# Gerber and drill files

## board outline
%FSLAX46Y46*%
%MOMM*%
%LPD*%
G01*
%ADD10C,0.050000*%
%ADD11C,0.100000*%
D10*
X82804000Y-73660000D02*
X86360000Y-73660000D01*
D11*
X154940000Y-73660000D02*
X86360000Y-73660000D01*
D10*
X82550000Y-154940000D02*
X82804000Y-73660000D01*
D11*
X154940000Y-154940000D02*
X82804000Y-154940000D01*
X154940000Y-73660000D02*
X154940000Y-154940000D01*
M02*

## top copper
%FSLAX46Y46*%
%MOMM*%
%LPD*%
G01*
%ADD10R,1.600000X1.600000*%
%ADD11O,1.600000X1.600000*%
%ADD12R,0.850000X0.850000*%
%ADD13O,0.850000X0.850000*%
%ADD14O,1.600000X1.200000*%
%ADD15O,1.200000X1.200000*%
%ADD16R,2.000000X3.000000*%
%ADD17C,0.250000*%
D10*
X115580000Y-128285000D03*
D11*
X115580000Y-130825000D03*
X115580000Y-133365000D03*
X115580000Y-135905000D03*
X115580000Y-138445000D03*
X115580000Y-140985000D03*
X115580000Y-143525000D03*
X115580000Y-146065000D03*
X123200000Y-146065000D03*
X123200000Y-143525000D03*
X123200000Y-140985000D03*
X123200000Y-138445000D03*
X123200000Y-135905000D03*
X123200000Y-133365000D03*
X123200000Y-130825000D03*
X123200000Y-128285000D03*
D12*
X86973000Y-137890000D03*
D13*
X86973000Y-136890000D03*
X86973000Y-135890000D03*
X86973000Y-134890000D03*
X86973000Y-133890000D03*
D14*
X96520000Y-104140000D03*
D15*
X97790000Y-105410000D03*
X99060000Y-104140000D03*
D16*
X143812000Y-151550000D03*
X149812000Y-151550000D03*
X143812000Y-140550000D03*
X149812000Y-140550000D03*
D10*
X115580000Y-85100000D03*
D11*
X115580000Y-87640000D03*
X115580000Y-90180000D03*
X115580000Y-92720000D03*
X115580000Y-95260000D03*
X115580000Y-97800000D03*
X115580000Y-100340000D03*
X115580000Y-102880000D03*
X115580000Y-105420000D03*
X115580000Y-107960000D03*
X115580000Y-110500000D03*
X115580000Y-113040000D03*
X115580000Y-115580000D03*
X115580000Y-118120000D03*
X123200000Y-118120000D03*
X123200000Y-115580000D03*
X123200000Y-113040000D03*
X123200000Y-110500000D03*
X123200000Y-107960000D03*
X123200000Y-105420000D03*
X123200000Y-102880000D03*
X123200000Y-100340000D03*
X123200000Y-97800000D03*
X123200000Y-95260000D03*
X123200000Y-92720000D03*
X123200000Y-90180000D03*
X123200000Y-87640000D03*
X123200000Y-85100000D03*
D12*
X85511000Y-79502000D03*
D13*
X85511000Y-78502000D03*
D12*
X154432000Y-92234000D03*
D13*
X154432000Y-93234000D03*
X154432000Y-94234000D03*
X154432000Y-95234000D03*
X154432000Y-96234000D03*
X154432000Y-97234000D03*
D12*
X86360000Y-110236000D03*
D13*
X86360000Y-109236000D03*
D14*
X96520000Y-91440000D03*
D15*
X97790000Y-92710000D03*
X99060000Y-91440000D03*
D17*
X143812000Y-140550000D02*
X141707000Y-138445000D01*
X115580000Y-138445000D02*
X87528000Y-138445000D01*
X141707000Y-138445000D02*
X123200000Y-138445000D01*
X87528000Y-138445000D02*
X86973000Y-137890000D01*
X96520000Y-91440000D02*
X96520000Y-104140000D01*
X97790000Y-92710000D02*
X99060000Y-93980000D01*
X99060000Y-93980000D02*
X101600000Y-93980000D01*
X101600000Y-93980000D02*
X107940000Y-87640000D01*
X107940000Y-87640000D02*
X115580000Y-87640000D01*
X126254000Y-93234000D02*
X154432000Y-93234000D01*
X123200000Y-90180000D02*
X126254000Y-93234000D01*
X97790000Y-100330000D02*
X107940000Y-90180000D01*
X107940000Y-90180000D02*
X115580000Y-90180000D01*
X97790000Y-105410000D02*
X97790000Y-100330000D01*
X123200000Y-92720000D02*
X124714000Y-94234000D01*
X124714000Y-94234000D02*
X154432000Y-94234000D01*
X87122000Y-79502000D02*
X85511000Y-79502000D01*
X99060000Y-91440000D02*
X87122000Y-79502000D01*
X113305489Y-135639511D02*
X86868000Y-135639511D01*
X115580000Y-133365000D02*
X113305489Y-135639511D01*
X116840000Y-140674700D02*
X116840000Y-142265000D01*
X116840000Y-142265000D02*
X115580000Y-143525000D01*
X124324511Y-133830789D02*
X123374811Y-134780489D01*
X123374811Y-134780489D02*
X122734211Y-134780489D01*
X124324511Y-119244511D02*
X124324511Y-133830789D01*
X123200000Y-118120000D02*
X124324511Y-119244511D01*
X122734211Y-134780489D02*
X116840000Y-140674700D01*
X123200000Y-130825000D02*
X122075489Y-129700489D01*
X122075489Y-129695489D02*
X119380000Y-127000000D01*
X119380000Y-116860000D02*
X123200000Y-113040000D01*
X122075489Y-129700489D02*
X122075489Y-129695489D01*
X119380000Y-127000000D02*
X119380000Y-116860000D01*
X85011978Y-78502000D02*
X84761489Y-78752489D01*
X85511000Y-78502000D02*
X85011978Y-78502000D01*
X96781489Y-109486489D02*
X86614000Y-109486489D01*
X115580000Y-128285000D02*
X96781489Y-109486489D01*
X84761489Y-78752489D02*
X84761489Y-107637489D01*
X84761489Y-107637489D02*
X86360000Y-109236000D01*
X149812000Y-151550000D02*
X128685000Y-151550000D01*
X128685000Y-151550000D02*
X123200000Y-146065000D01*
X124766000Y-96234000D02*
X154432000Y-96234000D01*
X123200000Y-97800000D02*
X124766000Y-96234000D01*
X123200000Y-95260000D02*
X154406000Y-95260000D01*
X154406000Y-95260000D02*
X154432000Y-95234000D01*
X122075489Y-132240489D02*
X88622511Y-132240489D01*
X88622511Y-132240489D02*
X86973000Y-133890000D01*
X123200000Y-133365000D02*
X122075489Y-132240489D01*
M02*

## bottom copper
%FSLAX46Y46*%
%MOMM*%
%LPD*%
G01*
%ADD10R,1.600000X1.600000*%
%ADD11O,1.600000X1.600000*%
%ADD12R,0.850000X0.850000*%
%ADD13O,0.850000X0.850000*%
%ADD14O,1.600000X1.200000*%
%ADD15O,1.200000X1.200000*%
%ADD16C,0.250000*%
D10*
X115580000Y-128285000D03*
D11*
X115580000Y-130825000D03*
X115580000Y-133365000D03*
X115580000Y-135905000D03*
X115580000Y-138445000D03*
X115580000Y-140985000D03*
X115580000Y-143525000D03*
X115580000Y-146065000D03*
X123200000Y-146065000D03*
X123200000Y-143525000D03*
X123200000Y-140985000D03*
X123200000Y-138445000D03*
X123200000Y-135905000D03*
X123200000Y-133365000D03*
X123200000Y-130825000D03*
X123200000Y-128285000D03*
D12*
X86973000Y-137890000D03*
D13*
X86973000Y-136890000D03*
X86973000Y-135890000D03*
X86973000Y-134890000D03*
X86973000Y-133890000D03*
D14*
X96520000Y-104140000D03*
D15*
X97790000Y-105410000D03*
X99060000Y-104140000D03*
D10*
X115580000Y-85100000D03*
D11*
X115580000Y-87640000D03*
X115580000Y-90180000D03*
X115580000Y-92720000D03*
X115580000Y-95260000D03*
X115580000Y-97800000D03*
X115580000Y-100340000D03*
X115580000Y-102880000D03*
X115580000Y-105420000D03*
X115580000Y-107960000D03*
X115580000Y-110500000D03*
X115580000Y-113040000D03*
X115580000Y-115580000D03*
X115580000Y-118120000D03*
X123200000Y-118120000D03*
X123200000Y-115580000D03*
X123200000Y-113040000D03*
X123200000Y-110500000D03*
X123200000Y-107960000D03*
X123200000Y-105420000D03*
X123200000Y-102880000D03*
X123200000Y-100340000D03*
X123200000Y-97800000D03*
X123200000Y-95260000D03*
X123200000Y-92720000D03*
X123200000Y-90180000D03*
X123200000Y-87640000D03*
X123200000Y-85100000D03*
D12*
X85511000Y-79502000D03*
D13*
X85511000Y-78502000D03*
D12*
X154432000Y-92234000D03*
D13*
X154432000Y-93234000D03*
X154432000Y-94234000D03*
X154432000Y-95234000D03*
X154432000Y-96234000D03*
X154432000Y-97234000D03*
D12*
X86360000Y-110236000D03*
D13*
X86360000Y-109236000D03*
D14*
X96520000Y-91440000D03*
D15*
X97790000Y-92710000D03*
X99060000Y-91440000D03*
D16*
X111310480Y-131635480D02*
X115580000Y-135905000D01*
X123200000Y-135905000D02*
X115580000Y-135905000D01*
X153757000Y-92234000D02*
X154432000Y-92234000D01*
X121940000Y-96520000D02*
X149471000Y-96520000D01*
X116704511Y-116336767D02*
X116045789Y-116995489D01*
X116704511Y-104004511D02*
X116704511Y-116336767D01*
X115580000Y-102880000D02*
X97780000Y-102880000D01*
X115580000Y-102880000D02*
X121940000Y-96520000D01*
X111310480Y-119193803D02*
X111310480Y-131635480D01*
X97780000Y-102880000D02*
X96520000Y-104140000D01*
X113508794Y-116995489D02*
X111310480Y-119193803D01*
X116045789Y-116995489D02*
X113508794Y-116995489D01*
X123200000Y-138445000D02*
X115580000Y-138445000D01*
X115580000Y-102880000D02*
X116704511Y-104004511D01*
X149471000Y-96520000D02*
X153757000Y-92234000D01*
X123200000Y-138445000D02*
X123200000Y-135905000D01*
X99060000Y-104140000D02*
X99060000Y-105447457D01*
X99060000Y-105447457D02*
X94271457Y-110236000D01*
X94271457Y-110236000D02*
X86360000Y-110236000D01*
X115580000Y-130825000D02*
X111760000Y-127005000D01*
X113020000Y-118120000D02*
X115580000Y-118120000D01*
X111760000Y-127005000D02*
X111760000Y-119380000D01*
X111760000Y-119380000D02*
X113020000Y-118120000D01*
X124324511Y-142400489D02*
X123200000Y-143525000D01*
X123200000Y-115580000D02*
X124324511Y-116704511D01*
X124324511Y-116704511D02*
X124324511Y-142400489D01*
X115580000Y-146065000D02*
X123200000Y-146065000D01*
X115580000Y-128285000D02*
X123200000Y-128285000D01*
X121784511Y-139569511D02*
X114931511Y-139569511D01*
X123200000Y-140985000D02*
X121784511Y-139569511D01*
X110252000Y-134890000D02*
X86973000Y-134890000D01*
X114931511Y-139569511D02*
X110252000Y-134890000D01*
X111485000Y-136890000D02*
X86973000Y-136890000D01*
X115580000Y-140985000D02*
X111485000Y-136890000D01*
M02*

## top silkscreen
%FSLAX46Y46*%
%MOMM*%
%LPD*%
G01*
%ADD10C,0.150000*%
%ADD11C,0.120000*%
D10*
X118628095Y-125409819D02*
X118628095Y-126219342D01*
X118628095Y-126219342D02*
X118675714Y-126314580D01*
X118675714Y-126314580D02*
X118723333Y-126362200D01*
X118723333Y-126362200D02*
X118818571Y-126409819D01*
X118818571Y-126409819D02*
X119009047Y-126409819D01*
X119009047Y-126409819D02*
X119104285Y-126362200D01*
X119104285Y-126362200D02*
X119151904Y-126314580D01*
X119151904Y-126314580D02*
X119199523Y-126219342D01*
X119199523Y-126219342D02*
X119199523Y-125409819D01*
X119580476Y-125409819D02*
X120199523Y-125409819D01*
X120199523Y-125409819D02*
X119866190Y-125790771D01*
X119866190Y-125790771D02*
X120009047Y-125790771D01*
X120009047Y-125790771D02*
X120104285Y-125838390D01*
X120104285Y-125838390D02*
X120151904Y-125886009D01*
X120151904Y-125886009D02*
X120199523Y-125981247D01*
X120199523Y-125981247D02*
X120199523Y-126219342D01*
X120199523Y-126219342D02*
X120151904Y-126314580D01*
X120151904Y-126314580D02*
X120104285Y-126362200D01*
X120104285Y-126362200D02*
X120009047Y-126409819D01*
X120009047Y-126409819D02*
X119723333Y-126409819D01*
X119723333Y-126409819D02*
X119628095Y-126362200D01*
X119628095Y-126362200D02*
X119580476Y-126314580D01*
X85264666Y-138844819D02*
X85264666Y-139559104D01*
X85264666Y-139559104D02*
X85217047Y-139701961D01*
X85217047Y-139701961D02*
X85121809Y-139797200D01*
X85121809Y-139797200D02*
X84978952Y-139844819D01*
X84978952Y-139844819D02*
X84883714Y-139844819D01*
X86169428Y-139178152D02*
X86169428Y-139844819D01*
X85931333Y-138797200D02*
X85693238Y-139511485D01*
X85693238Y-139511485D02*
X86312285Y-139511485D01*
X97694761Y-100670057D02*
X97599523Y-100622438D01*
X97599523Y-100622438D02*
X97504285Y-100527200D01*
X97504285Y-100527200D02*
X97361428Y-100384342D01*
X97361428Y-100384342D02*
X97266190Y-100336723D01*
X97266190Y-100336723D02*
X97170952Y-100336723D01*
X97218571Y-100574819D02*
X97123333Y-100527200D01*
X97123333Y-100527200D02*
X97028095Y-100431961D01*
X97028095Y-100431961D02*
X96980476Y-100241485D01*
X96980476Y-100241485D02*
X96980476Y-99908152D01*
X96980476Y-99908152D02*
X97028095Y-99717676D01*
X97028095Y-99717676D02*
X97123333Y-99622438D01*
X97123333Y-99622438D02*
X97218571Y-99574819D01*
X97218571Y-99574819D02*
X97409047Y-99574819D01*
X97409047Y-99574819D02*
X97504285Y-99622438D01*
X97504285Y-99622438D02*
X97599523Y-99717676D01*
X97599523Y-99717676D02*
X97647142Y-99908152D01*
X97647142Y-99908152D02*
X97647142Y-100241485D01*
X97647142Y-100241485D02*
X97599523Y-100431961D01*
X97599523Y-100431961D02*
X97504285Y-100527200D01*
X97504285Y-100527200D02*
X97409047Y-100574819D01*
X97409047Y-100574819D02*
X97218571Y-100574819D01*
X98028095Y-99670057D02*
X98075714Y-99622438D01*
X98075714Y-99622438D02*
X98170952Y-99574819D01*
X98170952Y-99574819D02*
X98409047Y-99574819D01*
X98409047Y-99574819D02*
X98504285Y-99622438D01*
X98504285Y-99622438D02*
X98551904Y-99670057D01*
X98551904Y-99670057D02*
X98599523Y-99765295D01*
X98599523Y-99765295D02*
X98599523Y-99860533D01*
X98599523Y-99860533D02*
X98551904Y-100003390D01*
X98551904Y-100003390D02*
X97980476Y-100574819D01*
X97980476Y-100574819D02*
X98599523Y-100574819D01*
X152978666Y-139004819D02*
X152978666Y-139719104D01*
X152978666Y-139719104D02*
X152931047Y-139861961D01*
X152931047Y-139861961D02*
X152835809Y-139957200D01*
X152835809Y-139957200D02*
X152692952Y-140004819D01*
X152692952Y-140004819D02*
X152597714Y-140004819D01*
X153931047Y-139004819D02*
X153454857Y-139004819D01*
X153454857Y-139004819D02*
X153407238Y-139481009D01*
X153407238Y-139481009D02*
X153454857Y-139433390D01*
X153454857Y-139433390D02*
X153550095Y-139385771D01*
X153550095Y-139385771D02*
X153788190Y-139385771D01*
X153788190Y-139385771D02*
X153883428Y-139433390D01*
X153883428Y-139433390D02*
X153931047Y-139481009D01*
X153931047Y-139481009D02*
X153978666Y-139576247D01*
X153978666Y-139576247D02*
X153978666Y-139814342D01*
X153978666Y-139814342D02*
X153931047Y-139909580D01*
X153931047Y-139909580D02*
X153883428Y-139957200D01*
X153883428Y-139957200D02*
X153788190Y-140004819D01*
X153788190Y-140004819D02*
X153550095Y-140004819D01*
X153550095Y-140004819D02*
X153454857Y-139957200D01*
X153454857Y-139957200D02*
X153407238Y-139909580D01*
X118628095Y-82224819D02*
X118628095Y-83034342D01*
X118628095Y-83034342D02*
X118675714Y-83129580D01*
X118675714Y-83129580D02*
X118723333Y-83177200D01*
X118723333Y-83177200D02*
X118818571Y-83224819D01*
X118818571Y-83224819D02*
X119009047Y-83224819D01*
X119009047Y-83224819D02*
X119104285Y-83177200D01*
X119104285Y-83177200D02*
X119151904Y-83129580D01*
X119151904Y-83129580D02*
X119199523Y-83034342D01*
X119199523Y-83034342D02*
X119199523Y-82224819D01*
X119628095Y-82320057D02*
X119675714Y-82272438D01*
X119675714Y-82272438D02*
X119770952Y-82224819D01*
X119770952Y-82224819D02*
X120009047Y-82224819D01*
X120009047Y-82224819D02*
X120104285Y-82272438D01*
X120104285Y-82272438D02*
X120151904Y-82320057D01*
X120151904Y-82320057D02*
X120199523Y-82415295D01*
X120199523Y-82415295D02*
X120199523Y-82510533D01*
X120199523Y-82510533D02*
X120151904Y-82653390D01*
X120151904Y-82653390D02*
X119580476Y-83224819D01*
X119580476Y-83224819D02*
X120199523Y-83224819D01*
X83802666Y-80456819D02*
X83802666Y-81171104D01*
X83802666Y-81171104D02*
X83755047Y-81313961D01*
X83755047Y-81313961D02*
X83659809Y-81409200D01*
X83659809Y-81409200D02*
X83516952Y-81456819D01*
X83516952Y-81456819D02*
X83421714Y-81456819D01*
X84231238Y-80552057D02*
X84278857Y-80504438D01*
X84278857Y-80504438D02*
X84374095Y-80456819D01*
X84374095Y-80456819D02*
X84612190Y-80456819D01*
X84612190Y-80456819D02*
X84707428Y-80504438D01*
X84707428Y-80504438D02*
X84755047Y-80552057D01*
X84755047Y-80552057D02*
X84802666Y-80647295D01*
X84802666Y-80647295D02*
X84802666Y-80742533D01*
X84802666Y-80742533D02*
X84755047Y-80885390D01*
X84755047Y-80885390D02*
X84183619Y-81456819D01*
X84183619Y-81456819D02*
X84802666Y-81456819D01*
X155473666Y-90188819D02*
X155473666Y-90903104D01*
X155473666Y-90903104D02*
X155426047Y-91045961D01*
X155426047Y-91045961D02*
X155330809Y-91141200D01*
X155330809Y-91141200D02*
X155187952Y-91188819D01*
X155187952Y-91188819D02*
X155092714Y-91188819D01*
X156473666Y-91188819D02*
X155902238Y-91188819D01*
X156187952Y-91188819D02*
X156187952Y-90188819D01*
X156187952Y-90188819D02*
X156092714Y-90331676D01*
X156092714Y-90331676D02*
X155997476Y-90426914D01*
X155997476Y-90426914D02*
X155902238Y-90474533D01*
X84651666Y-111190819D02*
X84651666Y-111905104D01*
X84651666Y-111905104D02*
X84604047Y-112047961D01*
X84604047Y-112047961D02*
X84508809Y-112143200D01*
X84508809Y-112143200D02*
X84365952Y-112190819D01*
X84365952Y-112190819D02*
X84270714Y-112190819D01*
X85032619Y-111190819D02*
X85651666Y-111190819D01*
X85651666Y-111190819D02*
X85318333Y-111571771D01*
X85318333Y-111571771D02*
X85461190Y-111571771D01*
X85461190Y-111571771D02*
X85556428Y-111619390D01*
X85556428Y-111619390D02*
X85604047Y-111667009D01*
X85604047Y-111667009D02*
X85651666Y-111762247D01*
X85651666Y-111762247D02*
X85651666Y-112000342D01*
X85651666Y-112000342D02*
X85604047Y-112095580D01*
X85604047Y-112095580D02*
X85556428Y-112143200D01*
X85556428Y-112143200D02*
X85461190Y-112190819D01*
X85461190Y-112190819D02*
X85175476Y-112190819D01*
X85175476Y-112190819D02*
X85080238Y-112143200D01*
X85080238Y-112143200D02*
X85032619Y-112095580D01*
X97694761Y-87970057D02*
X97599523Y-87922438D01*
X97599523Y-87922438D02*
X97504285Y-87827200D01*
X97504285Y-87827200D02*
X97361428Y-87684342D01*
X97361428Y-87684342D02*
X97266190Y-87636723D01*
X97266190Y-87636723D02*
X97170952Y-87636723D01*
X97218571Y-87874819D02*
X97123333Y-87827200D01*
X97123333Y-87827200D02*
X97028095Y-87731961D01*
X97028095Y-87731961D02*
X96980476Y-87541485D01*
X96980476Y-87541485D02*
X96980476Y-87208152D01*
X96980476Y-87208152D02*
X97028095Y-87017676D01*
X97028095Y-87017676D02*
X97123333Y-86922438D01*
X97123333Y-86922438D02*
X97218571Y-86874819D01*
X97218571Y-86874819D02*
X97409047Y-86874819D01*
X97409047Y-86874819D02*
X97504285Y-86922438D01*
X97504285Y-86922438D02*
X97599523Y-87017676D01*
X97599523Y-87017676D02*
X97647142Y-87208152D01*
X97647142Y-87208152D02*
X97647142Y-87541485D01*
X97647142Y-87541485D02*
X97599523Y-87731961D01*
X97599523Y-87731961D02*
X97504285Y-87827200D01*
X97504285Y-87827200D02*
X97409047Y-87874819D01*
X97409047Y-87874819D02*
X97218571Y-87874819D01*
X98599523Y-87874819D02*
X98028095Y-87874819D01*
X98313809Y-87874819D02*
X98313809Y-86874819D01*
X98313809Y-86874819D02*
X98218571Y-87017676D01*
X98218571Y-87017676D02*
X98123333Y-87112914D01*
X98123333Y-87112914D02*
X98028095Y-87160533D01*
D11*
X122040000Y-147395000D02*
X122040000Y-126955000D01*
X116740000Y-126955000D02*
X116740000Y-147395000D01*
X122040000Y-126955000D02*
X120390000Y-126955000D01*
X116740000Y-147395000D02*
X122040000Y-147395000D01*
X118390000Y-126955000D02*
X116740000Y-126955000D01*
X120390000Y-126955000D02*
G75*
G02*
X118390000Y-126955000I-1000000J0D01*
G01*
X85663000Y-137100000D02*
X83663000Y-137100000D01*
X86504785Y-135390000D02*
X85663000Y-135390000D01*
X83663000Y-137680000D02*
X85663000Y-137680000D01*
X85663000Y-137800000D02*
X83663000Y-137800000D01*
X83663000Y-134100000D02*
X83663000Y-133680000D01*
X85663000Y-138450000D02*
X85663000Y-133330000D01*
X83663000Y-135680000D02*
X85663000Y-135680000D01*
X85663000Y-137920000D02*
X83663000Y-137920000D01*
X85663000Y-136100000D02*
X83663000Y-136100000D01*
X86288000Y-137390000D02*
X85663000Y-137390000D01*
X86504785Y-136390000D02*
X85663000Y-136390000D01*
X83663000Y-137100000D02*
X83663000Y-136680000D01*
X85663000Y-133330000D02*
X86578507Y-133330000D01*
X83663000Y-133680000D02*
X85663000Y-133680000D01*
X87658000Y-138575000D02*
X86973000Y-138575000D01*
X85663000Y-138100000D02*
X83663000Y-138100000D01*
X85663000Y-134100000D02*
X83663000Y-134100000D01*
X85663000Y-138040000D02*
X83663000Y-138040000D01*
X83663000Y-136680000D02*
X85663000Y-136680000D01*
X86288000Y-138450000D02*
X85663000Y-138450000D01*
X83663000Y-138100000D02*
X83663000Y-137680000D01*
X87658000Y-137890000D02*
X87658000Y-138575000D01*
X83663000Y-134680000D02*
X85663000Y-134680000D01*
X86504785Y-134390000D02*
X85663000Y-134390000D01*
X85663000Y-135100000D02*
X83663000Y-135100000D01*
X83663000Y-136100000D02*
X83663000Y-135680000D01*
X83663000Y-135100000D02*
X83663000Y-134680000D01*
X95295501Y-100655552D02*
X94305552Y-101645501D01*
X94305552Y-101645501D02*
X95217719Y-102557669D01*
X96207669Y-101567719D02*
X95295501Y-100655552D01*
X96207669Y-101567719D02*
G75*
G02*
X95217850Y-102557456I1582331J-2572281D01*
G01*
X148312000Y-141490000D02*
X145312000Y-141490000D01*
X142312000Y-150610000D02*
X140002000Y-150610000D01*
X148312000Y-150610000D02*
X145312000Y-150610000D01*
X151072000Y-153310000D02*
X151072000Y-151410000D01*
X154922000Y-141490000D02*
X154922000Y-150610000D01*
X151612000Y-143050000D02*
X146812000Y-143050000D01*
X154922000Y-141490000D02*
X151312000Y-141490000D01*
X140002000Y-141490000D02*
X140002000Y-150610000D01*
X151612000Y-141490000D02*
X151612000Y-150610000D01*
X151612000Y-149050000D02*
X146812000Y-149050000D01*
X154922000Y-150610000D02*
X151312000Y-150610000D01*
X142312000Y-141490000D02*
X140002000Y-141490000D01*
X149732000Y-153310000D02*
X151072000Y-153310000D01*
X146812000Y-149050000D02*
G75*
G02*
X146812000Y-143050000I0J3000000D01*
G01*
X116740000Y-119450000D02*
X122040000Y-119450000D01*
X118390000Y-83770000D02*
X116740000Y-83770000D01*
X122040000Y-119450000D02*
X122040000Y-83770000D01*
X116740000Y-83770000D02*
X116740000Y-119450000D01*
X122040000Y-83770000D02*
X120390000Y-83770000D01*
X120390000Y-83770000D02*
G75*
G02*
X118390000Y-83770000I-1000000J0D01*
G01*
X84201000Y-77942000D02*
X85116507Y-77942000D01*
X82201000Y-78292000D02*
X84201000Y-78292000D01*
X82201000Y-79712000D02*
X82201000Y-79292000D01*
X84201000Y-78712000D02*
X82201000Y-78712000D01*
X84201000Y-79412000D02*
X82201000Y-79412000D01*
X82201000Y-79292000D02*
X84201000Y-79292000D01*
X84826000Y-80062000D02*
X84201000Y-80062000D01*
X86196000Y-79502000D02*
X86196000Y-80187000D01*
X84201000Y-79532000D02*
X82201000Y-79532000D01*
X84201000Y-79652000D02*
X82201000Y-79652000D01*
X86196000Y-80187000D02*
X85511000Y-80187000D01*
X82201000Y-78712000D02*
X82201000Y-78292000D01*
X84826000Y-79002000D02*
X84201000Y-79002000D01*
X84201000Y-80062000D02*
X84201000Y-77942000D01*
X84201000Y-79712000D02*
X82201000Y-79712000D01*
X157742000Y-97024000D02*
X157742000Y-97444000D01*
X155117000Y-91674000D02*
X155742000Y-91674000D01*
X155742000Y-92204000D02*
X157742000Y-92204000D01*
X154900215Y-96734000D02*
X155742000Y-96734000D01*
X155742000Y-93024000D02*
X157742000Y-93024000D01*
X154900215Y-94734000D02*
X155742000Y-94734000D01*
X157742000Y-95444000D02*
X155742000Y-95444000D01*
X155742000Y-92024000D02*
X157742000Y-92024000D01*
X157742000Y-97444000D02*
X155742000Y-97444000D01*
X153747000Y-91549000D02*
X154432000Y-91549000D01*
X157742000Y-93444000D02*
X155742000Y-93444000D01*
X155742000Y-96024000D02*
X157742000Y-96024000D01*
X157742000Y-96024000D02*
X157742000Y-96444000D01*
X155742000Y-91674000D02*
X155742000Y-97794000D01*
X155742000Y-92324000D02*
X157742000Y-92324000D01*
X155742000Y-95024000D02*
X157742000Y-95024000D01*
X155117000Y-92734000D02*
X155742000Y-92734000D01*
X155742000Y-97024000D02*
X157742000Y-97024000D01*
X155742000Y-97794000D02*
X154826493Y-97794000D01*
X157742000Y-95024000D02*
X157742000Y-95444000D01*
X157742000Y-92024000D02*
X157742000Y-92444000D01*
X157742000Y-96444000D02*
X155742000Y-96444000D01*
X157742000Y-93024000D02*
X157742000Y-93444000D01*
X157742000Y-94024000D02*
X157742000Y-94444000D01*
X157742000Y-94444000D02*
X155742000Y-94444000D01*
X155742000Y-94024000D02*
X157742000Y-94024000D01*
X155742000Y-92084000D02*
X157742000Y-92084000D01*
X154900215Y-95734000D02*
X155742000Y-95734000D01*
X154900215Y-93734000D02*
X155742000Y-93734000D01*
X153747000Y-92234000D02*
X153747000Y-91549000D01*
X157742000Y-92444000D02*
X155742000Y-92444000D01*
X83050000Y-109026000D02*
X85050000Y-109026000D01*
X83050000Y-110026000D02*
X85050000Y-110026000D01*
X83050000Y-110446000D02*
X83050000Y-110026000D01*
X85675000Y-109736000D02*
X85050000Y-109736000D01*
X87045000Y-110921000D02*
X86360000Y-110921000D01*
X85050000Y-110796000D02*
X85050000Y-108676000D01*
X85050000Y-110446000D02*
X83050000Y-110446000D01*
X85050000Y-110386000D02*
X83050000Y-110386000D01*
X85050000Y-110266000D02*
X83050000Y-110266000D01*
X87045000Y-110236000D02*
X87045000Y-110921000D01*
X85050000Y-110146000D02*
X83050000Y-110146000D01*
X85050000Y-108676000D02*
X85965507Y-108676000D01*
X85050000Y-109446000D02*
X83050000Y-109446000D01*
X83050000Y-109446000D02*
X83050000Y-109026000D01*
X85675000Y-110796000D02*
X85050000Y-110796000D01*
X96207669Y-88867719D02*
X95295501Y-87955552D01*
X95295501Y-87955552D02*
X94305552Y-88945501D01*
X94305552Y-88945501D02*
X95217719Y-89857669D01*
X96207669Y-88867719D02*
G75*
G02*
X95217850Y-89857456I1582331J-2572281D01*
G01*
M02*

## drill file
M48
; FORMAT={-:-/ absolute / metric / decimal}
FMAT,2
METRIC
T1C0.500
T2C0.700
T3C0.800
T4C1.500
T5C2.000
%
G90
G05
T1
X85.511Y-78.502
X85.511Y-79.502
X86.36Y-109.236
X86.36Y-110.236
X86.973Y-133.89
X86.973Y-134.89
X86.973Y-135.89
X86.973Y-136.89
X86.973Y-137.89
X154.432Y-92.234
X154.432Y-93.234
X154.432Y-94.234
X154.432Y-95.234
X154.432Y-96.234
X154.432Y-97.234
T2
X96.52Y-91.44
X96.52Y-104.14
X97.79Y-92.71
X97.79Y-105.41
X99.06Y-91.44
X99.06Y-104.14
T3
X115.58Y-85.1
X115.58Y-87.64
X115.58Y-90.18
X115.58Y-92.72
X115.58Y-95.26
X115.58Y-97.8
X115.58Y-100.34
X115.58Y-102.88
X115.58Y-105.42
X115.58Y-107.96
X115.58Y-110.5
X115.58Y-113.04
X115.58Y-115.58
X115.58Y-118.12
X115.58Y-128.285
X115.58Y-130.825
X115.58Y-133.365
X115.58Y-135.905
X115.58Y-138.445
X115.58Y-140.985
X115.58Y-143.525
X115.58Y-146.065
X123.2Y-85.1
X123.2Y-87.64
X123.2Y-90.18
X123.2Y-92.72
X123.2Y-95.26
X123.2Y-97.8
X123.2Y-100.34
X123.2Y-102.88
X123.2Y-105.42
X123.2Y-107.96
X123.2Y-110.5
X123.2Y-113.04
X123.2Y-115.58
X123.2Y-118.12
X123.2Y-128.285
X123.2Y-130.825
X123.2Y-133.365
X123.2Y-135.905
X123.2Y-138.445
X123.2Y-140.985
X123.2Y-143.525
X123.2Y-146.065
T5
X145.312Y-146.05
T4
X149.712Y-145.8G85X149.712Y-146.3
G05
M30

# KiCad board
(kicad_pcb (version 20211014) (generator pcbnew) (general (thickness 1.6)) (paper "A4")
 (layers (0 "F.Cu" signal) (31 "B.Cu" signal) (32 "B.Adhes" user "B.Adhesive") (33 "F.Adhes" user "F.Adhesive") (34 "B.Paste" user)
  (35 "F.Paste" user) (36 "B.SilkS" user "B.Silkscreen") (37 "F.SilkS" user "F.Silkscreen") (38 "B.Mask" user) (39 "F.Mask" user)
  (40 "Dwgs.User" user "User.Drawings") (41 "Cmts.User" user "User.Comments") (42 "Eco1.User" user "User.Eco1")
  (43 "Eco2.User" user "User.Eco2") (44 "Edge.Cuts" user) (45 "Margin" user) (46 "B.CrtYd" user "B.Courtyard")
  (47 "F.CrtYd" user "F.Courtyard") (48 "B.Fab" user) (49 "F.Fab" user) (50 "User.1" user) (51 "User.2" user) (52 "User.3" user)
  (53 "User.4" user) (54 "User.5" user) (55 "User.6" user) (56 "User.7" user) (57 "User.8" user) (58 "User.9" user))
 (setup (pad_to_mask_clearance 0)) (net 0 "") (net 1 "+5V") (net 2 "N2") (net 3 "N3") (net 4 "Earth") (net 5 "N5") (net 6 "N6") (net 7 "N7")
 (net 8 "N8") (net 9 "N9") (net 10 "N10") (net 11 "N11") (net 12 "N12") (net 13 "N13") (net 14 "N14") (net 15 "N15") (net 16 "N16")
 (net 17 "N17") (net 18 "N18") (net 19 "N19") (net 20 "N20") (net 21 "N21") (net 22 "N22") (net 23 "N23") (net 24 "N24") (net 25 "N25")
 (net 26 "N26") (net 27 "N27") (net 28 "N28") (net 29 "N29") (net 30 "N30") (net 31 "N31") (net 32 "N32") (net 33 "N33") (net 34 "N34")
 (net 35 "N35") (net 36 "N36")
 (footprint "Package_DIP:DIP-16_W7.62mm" (layer "F.Cu") (at 115.58 128.285)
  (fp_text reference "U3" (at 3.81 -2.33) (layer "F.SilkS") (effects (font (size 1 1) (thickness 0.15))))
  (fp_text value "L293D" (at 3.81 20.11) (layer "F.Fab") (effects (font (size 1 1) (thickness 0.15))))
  (fp_line (start 6.46 19.11) (end 6.46 -1.33) (layer "F.SilkS") (width 0.12))
  (fp_line (start 1.16 -1.33) (end 1.16 19.11) (layer "F.SilkS") (width 0.12))
  (fp_line (start 6.46 -1.33) (end 4.81 -1.33) (layer "F.SilkS") (width 0.12))
  (fp_line (start 1.16 19.11) (end 6.46 19.11) (layer "F.SilkS") (width 0.12))
  (fp_line (start 2.81 -1.33) (end 1.16 -1.33) (layer "F.SilkS") (width 0.12))
  (fp_arc (start 4.81 -1.33) (mid 3.81 -0.33) (end 2.81 -1.33) (layer "F.SilkS") (width 0.12))
  (pad "1" thru_hole rect (at 0 0) (size 1.6 1.6) (drill 0.8) (layers *.Cu *.Mask) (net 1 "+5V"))
  (pad "2" thru_hole oval (at 0 2.54) (size 1.6 1.6) (drill 0.8) (layers *.Cu *.Mask) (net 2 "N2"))
  (pad "3" thru_hole oval (at 0 5.08) (size 1.6 1.6) (drill 0.8) (layers *.Cu *.Mask) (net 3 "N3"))
  (pad "4" thru_hole oval (at 0 7.62) (size 1.6 1.6) (drill 0.8) (layers *.Cu *.Mask) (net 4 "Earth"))
  (pad "5" thru_hole oval (at 0 10.16) (size 1.6 1.6) (drill 0.8) (layers *.Cu *.Mask) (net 4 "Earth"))
  (pad "6" thru_hole oval (at 0 12.7) (size 1.6 1.6) (drill 0.8) (layers *.Cu *.Mask) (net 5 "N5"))
  (pad "7" thru_hole oval (at 0 15.24) (size 1.6 1.6) (drill 0.8) (layers *.Cu *.Mask) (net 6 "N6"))
  (pad "8" thru_hole oval (at 0 17.78) (size 1.6 1.6) (drill 0.8) (layers *.Cu *.Mask) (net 1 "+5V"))
  (pad "9" thru_hole oval (at 7.62 17.78) (size 1.6 1.6) (drill 0.8) (layers *.Cu *.Mask) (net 1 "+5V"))
  (pad "10" thru_hole oval (at 7.62 15.24) (size 1.6 1.6) (drill 0.8) (layers *.Cu *.Mask) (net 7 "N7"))
  (pad "11" thru_hole oval (at 7.62 12.7) (size 1.6 1.6) (drill 0.8) (layers *.Cu *.Mask) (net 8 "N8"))
  (pad "12" thru_hole oval (at 7.62 10.16) (size 1.6 1.6) (drill 0.8) (layers *.Cu *.Mask) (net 4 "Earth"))
  (pad "13" thru_hole oval (at 7.62 7.62) (size 1.6 1.6) (drill 0.8) (layers *.Cu *.Mask) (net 4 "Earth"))
  (pad "14" thru_hole oval (at 7.62 5.08) (size 1.6 1.6) (drill 0.8) (layers *.Cu *.Mask) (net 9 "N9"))
  (pad "15" thru_hole oval (at 7.62 2.54) (size 1.6 1.6) (drill 0.8) (layers *.Cu *.Mask) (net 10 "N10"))
  (pad "16" thru_hole oval (at 7.62 0) (size 1.6 1.6) (drill 0.8) (layers *.Cu *.Mask) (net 1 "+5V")))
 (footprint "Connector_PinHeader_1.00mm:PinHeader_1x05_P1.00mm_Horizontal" (layer "F.Cu") (at 86.973 137.89 180)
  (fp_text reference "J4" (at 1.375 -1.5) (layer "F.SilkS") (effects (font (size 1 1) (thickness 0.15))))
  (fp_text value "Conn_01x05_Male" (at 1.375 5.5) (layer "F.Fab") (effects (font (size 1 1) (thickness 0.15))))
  (fp_line (start 1.31 0.79) (end 3.31 0.79) (layer "F.SilkS") (width 0.12))
  (fp_line (start 0.468215 2.5) (end 1.31 2.5) (layer "F.SilkS") (width 0.12))
  (fp_line (start 3.31 0.21) (end 1.31 0.21) (layer "F.SilkS") (width 0.12))
  (fp_line (start 1.31 0.09) (end 3.31 0.09) (layer "F.SilkS") (width 0.12))
  (fp_line (start 3.31 3.79) (end 3.31 4.21) (layer "F.SilkS") (width 0.12))
  (fp_line (start 1.31 -0.56) (end 1.31 4.56) (layer "F.SilkS") (width 0.12))
  (fp_line (start 3.31 2.21) (end 1.31 2.21) (layer "F.SilkS") (width 0.12))
  (fp_line (start 1.31 -0.03) (end 3.31 -0.03) (layer "F.SilkS") (width 0.12))
  (fp_line (start 1.31 1.79) (end 3.31 1.79) (layer "F.SilkS") (width 0.12))
  (fp_line (start 0.685 0.5) (end 1.31 0.5) (layer "F.SilkS") (width 0.12))
  (fp_line (start 0.468215 1.5) (end 1.31 1.5) (layer "F.SilkS") (width 0.12))
  (fp_line (start 3.31 0.79) (end 3.31 1.21) (layer "F.SilkS") (width 0.12))
  (fp_line (start 1.31 4.56) (end 0.394493 4.56) (layer "F.SilkS") (width 0.12))
  (fp_line (start 3.31 4.21) (end 1.31 4.21) (layer "F.SilkS") (width 0.12))
  (fp_line (start -0.685 -0.685) (end 0 -0.685) (layer "F.SilkS") (width 0.12))
  (fp_line (start 1.31 -0.21) (end 3.31 -0.21) (layer "F.SilkS") (width 0.12))
  (fp_line (start 1.31 3.79) (end 3.31 3.79) (layer "F.SilkS") (width 0.12))
  (fp_line (start 1.31 -0.15) (end 3.31 -0.15) (layer "F.SilkS") (width 0.12))
  (fp_line (start 3.31 1.21) (end 1.31 1.21) (layer "F.SilkS") (width 0.12))
  (fp_line (start 0.685 -0.56) (end 1.31 -0.56) (layer "F.SilkS") (width 0.12))
  (fp_line (start 3.31 -0.21) (end 3.31 0.21) (layer "F.SilkS") (width 0.12))
  (fp_line (start -0.685 0) (end -0.685 -0.685) (layer "F.SilkS") (width 0.12))
  (fp_line (start 3.31 3.21) (end 1.31 3.21) (layer "F.SilkS") (width 0.12))
  (fp_line (start 0.468215 3.5) (end 1.31 3.5) (layer "F.SilkS") (width 0.12))
  (fp_line (start 1.31 2.79) (end 3.31 2.79) (layer "F.SilkS") (width 0.12))
  (fp_line (start 3.31 1.79) (end 3.31 2.21) (layer "F.SilkS") (width 0.12))
  (fp_line (start 3.31 2.79) (end 3.31 3.21) (layer "F.SilkS") (width 0.12))
  (pad "1" thru_hole rect (at 0 0 180) (size 0.85 0.85) (drill 0.5) (layers *.Cu *.Mask) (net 4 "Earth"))
  (pad "2" thru_hole oval (at 0 1 180) (size 0.85 0.85) (drill 0.5) (layers *.Cu *.Mask) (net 5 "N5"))
  (pad "3" thru_hole oval (at 0 2 180) (size 0.85 0.85) (drill 0.5) (layers *.Cu *.Mask) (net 3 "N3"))
  (pad "4" thru_hole oval (at 0 3 180) (size 0.85 0.85) (drill 0.5) (layers *.Cu *.Mask) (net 8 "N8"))
  (pad "5" thru_hole oval (at 0 4 180) (size 0.85 0.85) (drill 0.5) (layers *.Cu *.Mask) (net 9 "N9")))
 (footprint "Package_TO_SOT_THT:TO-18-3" (layer "F.Cu") (at 96.52 104.14)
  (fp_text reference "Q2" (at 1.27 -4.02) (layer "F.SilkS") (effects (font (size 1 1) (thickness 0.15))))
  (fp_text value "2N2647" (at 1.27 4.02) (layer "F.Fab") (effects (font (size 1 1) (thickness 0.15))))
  (fp_line (start -1.224499 -3.484448) (end -2.214448 -2.494499) (layer "F.SilkS") (width 0.12))
  (fp_line (start -2.214448 -2.494499) (end -1.302281 -1.582331) (layer "F.SilkS") (width 0.12))
  (fp_line (start -0.312331 -2.572281) (end -1.224499 -3.484448) (layer "F.SilkS") (width 0.12))
  (fp_arc (start -0.312331 -2.572281) (mid 3.405374 2.135551) (end -1.30215 -1.582544) (layer "F.SilkS") (width 0.12))
  (pad "1" thru_hole oval (at 0 0) (size 1.6 1.2) (drill 0.7) (layers *.Cu *.Mask) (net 4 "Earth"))
  (pad "2" thru_hole oval (at 1.27 1.27) (size 1.2 1.2) (drill 0.7) (layers *.Cu *.Mask) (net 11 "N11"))
  (pad "3" thru_hole oval (at 2.54 0) (size 1.2 1.2) (drill 0.7) (layers *.Cu *.Mask) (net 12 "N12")))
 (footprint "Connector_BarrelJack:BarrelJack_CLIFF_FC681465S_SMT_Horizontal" (layer "F.Cu") (at 146.812 146.05 180)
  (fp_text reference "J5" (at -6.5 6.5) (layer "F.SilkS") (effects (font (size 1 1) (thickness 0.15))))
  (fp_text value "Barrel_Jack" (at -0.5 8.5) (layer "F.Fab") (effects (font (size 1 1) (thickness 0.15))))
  (fp_line (start -1.5 4.56) (end 1.5 4.56) (layer "F.SilkS") (width 0.12))
  (fp_line (start 4.5 -4.56) (end 6.81 -4.56) (layer "F.SilkS") (width 0.12))
  (fp_line (start -1.5 -4.56) (end 1.5 -4.56) (layer "F.SilkS") (width 0.12))
  (fp_line (start -4.26 -7.26) (end -4.26 -5.36) (layer "F.SilkS") (width 0.12))
  (fp_line (start -8.11 4.56) (end -8.11 -4.56) (layer "F.SilkS") (width 0.12))
  (fp_line (start -4.8 3) (end 0 3) (layer "F.SilkS") (width 0.12))
  (fp_line (start -8.11 4.56) (end -4.5 4.56) (layer "F.SilkS") (width 0.12))
  (fp_line (start 6.81 4.56) (end 6.81 -4.56) (layer "F.SilkS") (width 0.12))
  (fp_line (start -4.8 4.56) (end -4.8 -4.56) (layer "F.SilkS") (width 0.12))
  (fp_line (start -4.8 -3) (end 0 -3) (layer "F.SilkS") (width 0.12))
  (fp_line (start -8.11 -4.56) (end -4.5 -4.56) (layer "F.SilkS") (width 0.12))
  (fp_line (start 4.5 4.56) (end 6.81 4.56) (layer "F.SilkS") (width 0.12))
  (fp_line (start -2.92 -7.26) (end -4.26 -7.26) (layer "F.SilkS") (width 0.12))
  (fp_arc (start 0 -3) (mid 3 0) (end 0 3) (layer "F.SilkS") (width 0.12))
  (pad "" np_thru_hole circle (at 1.5 0 270) (size 2 2) (drill 2) (layers *.Cu *.Mask))
  (pad "" np_thru_hole oval (at -2.9 0 270) (size 2 1.5) (drill oval 2 1.5) (layers *.Cu *.Mask))
  (pad "1" smd rect (at 3 -5.5 270) (size 3 2) (layers "F.Cu" "F.Paste" "F.Mask") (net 1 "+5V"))
  (pad "1" smd rect (at -3 -5.5 270) (size 3 2) (layers "F.Cu" "F.Paste" "F.Mask") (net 1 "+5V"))
  (pad "2" smd rect (at 3 5.5 270) (size 3 2) (layers "F.Cu" "F.Paste" "F.Mask") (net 4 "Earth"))
  (pad "3" smd rect (at -3 5.5 270) (size 3 2) (layers "F.Cu" "F.Paste" "F.Mask")))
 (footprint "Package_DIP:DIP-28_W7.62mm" (layer "F.Cu") (at 115.58 85.1)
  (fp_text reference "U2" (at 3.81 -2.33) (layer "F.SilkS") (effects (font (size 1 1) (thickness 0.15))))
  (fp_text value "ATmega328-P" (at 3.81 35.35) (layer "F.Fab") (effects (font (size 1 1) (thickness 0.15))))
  (fp_line (start 1.16 34.35) (end 6.46 34.35) (layer "F.SilkS") (width 0.12))
  (fp_line (start 2.81 -1.33) (end 1.16 -1.33) (layer "F.SilkS") (width 0.12))
  (fp_line (start 6.46 34.35) (end 6.46 -1.33) (layer "F.SilkS") (width 0.12))
  (fp_line (start 1.16 -1.33) (end 1.16 34.35) (layer "F.SilkS") (width 0.12))
  (fp_line (start 6.46 -1.33) (end 4.81 -1.33) (layer "F.SilkS") (width 0.12))
  (fp_arc (start 4.81 -1.33) (mid 3.81 -0.33) (end 2.81 -1.33) (layer "F.SilkS") (width 0.12))
  (pad "1" thru_hole rect (at 0 0) (size 1.6 1.6) (drill 0.8) (layers *.Cu *.Mask) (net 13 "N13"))
  (pad "2" thru_hole oval (at 0 2.54) (size 1.6 1.6) (drill 0.8) (layers *.Cu *.Mask) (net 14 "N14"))
  (pad "3" thru_hole oval (at 0 5.08) (size 1.6 1.6) (drill 0.8) (layers *.Cu *.Mask) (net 11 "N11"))
  (pad "4" thru_hole oval (at 0 7.62) (size 1.6 1.6) (drill 0.8) (layers *.Cu *.Mask) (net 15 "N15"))
  (pad "5" thru_hole oval (at 0 10.16) (size 1.6 1.6) (drill 0.8) (layers *.Cu *.Mask) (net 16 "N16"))
  (pad "6" thru_hole oval (at 0 12.7) (size 1.6 1.6) (drill 0.8) (layers *.Cu *.Mask) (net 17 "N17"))
  (pad "7" thru_hole oval (at 0 15.24) (size 1.6 1.6) (drill 0.8) (layers *.Cu *.Mask) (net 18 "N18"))
  (pad "8" thru_hole oval (at 0 17.78) (size 1.6 1.6) (drill 0.8) (layers *.Cu *.Mask) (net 4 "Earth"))
  (pad "9" thru_hole oval (at 0 20.32) (size 1.6 1.6) (drill 0.8) (layers *.Cu *.Mask) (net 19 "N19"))
  (pad "10" thru_hole oval (at 0 22.86) (size 1.6 1.6) (drill 0.8) (layers *.Cu *.Mask) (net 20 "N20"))
  (pad "11" thru_hole oval (at 0 25.4) (size 1.6 1.6) (drill 0.8) (layers *.Cu *.Mask) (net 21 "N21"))
  (pad "12" thru_hole oval (at 0 27.94) (size 1.6 1.6) (drill 0.8) (layers *.Cu *.Mask) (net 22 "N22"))
  (pad "13" thru_hole oval (at 0 30.48) (size 1.6 1.6) (drill 0.8) (layers *.Cu *.Mask) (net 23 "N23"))
  (pad "14" thru_hole oval (at 0 33.02) (size 1.6 1.6) (drill 0.8) (layers *.Cu *.Mask) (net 2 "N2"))
  (pad "15" thru_hole oval (at 7.62 33.02) (size 1.6 1.6) (drill 0.8) (layers *.Cu *.Mask) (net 6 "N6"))
  (pad "16" thru_hole oval (at 7.62 30.48) (size 1.6 1.6) (drill 0.8) (layers *.Cu *.Mask) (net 7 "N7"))
  (pad "17" thru_hole oval (at 7.62 27.94) (size 1.6 1.6) (drill 0.8) (layers *.Cu *.Mask) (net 10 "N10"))
  (pad "18" thru_hole oval (at 7.62 25.4) (size 1.6 1.6) (drill 0.8) (layers *.Cu *.Mask) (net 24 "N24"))
  (pad "19" thru_hole oval (at 7.62 22.86) (size 1.6 1.6) (drill 0.8) (layers *.Cu *.Mask) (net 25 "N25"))
  (pad "20" thru_hole oval (at 7.62 20.32) (size 1.6 1.6) (drill 0.8) (layers *.Cu *.Mask) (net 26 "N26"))
  (pad "21" thru_hole oval (at 7.62 17.78) (size 1.6 1.6) (drill 0.8) (layers *.Cu *.Mask) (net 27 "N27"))
  (pad "22" thru_hole oval (at 7.62 15.24) (size 1.6 1.6) (drill 0.8) (layers *.Cu *.Mask) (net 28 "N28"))
  (pad "23" thru_hole oval (at 7.62 12.7) (size 1.6 1.6) (drill 0.8) (layers *.Cu *.Mask) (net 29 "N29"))
  (pad "24" thru_hole oval (at 7.62 10.16) (size 1.6 1.6) (drill 0.8) (layers *.Cu *.Mask) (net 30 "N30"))
  (pad "25" thru_hole oval (at 7.62 7.62) (size 1.6 1.6) (drill 0.8) (layers *.Cu *.Mask) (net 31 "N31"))
  (pad "26" thru_hole oval (at 7.62 5.08) (size 1.6 1.6) (drill 0.8) (layers *.Cu *.Mask) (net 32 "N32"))
  (pad "27" thru_hole oval (at 7.62 2.54) (size 1.6 1.6) (drill 0.8) (layers *.Cu *.Mask) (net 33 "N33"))
  (pad "28" thru_hole oval (at 7.62 0) (size 1.6 1.6) (drill 0.8) (layers *.Cu *.Mask) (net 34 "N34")))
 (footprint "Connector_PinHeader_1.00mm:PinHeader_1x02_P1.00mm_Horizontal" (layer "F.Cu") (at 85.511 79.502 180)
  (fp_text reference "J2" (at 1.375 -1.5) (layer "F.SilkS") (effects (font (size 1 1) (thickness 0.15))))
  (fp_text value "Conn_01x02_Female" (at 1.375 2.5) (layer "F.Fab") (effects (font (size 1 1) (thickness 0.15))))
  (fp_line (start 1.31 1.56) (end 0.394493 1.56) (layer "F.SilkS") (width 0.12))
  (fp_line (start 3.31 1.21) (end 1.31 1.21) (layer "F.SilkS") (width 0.12))
  (fp_line (start 3.31 -0.21) (end 3.31 0.21) (layer "F.SilkS") (width 0.12))
  (fp_line (start 1.31 0.79) (end 3.31 0.79) (layer "F.SilkS") (width 0.12))
  (fp_line (start 1.31 0.09) (end 3.31 0.09) (layer "F.SilkS") (width 0.12))
  (fp_line (start 3.31 0.21) (end 1.31 0.21) (layer "F.SilkS") (width 0.12))
  (fp_line (start 0.685 -0.56) (end 1.31 -0.56) (layer "F.SilkS") (width 0.12))
  (fp_line (start -0.685 0) (end -0.685 -0.685) (layer "F.SilkS") (width 0.12))
  (fp_line (start 1.31 -0.03) (end 3.31 -0.03) (layer "F.SilkS") (width 0.12))
  (fp_line (start 1.31 -0.15) (end 3.31 -0.15) (layer "F.SilkS") (width 0.12))
  (fp_line (start -0.685 -0.685) (end 0 -0.685) (layer "F.SilkS") (width 0.12))
  (fp_line (start 3.31 0.79) (end 3.31 1.21) (layer "F.SilkS") (width 0.12))
  (fp_line (start 0.685 0.5) (end 1.31 0.5) (layer "F.SilkS") (width 0.12))
  (fp_line (start 1.31 -0.56) (end 1.31 1.56) (layer "F.SilkS") (width 0.12))
  (fp_line (start 1.31 -0.21) (end 3.31 -0.21) (layer "F.SilkS") (width 0.12))
  (pad "1" thru_hole rect (at 0 0 180) (size 0.85 0.85) (drill 0.5) (layers *.Cu *.Mask) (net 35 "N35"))
  (pad "2" thru_hole oval (at 0 1 180) (size 0.85 0.85) (drill 0.5) (layers *.Cu *.Mask) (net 1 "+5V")))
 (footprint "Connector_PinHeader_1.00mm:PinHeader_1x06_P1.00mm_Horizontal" (layer "F.Cu") (at 154.432 92.234)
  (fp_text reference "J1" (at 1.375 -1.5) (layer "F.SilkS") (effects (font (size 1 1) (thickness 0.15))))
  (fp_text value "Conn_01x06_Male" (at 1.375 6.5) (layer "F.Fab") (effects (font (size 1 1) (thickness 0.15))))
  (fp_line (start 3.31 4.79) (end 3.31 5.21) (layer "F.SilkS") (width 0.12))
  (fp_line (start 0.685 -0.56) (end 1.31 -0.56) (layer "F.SilkS") (width 0.12))
  (fp_line (start 1.31 -0.03) (end 3.31 -0.03) (layer "F.SilkS") (width 0.12))
  (fp_line (start 0.468215 4.5) (end 1.31 4.5) (layer "F.SilkS") (width 0.12))
  (fp_line (start 1.31 0.79) (end 3.31 0.79) (layer "F.SilkS") (width 0.12))
  (fp_line (start 0.468215 2.5) (end 1.31 2.5) (layer "F.SilkS") (width 0.12))
  (fp_line (start 3.31 3.21) (end 1.31 3.21) (layer "F.SilkS") (width 0.12))
  (fp_line (start 1.31 -0.21) (end 3.31 -0.21) (layer "F.SilkS") (width 0.12))
  (fp_line (start 3.31 5.21) (end 1.31 5.21) (layer "F.SilkS") (width 0.12))
  (fp_line (start -0.685 -0.685) (end 0 -0.685) (layer "F.SilkS") (width 0.12))
  (fp_line (start 3.31 1.21) (end 1.31 1.21) (layer "F.SilkS") (width 0.12))
  (fp_line (start 1.31 3.79) (end 3.31 3.79) (layer "F.SilkS") (width 0.12))
  (fp_line (start 3.31 3.79) (end 3.31 4.21) (layer "F.SilkS") (width 0.12))
  (fp_line (start 1.31 -0.56) (end 1.31 5.56) (layer "F.SilkS") (width 0.12))
  (fp_line (start 1.31 0.09) (end 3.31 0.09) (layer "F.SilkS") (width 0.12))
  (fp_line (start 1.31 2.79) (end 3.31 2.79) (layer "F.SilkS") (width 0.12))
  (fp_line (start 0.685 0.5) (end 1.31 0.5) (layer "F.SilkS") (width 0.12))
  (fp_line (start 1.31 4.79) (end 3.31 4.79) (layer "F.SilkS") (width 0.12))
  (fp_line (start 1.31 5.56) (end 0.394493 5.56) (layer "F.SilkS") (width 0.12))
  (fp_line (start 3.31 2.79) (end 3.31 3.21) (layer "F.SilkS") (width 0.12))
  (fp_line (start 3.31 -0.21) (end 3.31 0.21) (layer "F.SilkS") (width 0.12))
  (fp_line (start 3.31 4.21) (end 1.31 4.21) (layer "F.SilkS") (width 0.12))
  (fp_line (start 3.31 0.79) (end 3.31 1.21) (layer "F.SilkS") (width 0.12))
  (fp_line (start 3.31 1.79) (end 3.31 2.21) (layer "F.SilkS") (width 0.12))
  (fp_line (start 3.31 2.21) (end 1.31 2.21) (layer "F.SilkS") (width 0.12))
  (fp_line (start 1.31 1.79) (end 3.31 1.79) (layer "F.SilkS") (width 0.12))
  (fp_line (start 1.31 -0.15) (end 3.31 -0.15) (layer "F.SilkS") (width 0.12))
  (fp_line (start 0.468215 3.5) (end 1.31 3.5) (layer "F.SilkS") (width 0.12))
  (fp_line (start 0.468215 1.5) (end 1.31 1.5) (layer "F.SilkS") (width 0.12))
  (fp_line (start -0.685 0) (end -0.685 -0.685) (layer "F.SilkS") (width 0.12))
  (fp_line (start 3.31 0.21) (end 1.31 0.21) (layer "F.SilkS") (width 0.12))
  (pad "1" thru_hole rect (at 0 0) (size 0.85 0.85) (drill 0.5) (layers *.Cu *.Mask) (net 4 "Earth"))
  (pad "2" thru_hole oval (at 0 1) (size 0.85 0.85) (drill 0.5) (layers *.Cu *.Mask) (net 32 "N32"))
  (pad "3" thru_hole oval (at 0 2) (size 0.85 0.85) (drill 0.5) (layers *.Cu *.Mask) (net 31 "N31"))
  (pad "4" thru_hole oval (at 0 3) (size 0.85 0.85) (drill 0.5) (layers *.Cu *.Mask) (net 30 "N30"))
  (pad "5" thru_hole oval (at 0 4) (size 0.85 0.85) (drill 0.5) (layers *.Cu *.Mask) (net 29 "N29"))
  (pad "6" thru_hole oval (at 0 5) (size 0.85 0.85) (drill 0.5) (layers *.Cu *.Mask) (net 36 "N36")))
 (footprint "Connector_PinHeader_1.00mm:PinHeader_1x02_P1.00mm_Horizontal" (layer "F.Cu") (at 86.36 110.236 180)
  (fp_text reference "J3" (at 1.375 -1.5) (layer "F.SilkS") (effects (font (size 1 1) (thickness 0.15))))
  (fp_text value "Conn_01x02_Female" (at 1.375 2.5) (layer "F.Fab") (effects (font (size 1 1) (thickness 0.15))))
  (fp_line (start 3.31 1.21) (end 1.31 1.21) (layer "F.SilkS") (width 0.12))
  (fp_line (start 3.31 0.21) (end 1.31 0.21) (layer "F.SilkS") (width 0.12))
  (fp_line (start 3.31 -0.21) (end 3.31 0.21) (layer "F.SilkS") (width 0.12))
  (fp_line (start 0.685 0.5) (end 1.31 0.5) (layer "F.SilkS") (width 0.12))
  (fp_line (start -0.685 -0.685) (end 0 -0.685) (layer "F.SilkS") (width 0.12))
  (fp_line (start 1.31 -0.56) (end 1.31 1.56) (layer "F.SilkS") (width 0.12))
  (fp_line (start 1.31 -0.21) (end 3.31 -0.21) (layer "F.SilkS") (width 0.12))
  (fp_line (start 1.31 -0.15) (end 3.31 -0.15) (layer "F.SilkS") (width 0.12))
  (fp_line (start 1.31 -0.03) (end 3.31 -0.03) (layer "F.SilkS") (width 0.12))
  (fp_line (start -0.685 0) (end -0.685 -0.685) (layer "F.SilkS") (width 0.12))
  (fp_line (start 1.31 0.09) (end 3.31 0.09) (layer "F.SilkS") (width 0.12))
  (fp_line (start 1.31 1.56) (end 0.394493 1.56) (layer "F.SilkS") (width 0.12))
  (fp_line (start 1.31 0.79) (end 3.31 0.79) (layer "F.SilkS") (width 0.12))
  (fp_line (start 3.31 0.79) (end 3.31 1.21) (layer "F.SilkS") (width 0.12))
  (fp_line (start 0.685 -0.56) (end 1.31 -0.56) (layer "F.SilkS") (width 0.12))
  (pad "1" thru_hole rect (at 0 0 180) (size 0.85 0.85) (drill 0.5) (layers *.Cu *.Mask) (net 12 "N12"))
  (pad "2" thru_hole oval (at 0 1 180) (size 0.85 0.85) (drill 0.5) (layers *.Cu *.Mask) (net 1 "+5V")))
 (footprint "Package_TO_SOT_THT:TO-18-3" (layer "F.Cu") (at 96.52 91.44)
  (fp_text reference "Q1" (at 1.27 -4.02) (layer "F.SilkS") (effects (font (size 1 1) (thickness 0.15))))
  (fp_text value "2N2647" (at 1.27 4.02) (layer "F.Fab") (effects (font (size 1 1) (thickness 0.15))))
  (fp_line (start -0.312331 -2.572281) (end -1.224499 -3.484448) (layer "F.SilkS") (width 0.12))
  (fp_line (start -1.224499 -3.484448) (end -2.214448 -2.494499) (layer "F.SilkS") (width 0.12))
  (fp_line (start -2.214448 -2.494499) (end -1.302281 -1.582331) (layer "F.SilkS") (width 0.12))
  (fp_arc (start -0.312331 -2.572281) (mid 3.405374 2.135551) (end -1.30215 -1.582544) (layer "F.SilkS") (width 0.12))
  (pad "1" thru_hole oval (at 0 0) (size 1.6 1.2) (drill 0.7) (layers *.Cu *.Mask) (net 4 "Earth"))
  (pad "2" thru_hole oval (at 1.27 1.27) (size 1.2 1.2) (drill 0.7) (layers *.Cu *.Mask) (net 14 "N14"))
  (pad "3" thru_hole oval (at 2.54 0) (size 1.2 1.2) (drill 0.7) (layers *.Cu *.Mask) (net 35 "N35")))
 (gr_line (start 82.804 73.66) (end 86.36 73.66) (layer "Edge.Cuts") (width 0.05))
 (gr_line (start 154.94 73.66) (end 86.36 73.66) (layer "Edge.Cuts") (width 0.1))
 (gr_line (start 82.55 154.94) (end 82.804 73.66) (layer "Edge.Cuts") (width 0.05))
 (gr_line (start 154.94 154.94) (end 82.804 154.94) (layer "Edge.Cuts") (width 0.1))
 (gr_line (start 154.94 73.66) (end 154.94 154.94) (layer "Edge.Cuts") (width 0.1))
 (segment (start 143.812 140.55) (end 141.707 138.445) (width 0.25) (layer "F.Cu") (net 4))
 (segment (start 115.58 138.445) (end 87.528 138.445) (width 0.25) (layer "F.Cu") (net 4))
 (segment (start 141.707 138.445) (end 123.2 138.445) (width 0.25) (layer "F.Cu") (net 4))
 (segment (start 87.528 138.445) (end 86.973 137.89) (width 0.25) (layer "F.Cu") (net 4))
 (segment (start 96.52 91.44) (end 96.52 104.14) (width 0.25) (layer "F.Cu") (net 4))
 (segment (start 111.31048 131.63548) (end 115.58 135.905) (width 0.25) (layer "B.Cu") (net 4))
 (segment (start 123.2 135.905) (end 115.58 135.905) (width 0.25) (layer "B.Cu") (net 4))
 (segment (start 153.757 92.234) (end 154.432 92.234) (width 0.25) (layer "B.Cu") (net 4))
 (segment (start 121.94 96.52) (end 149.471 96.52) (width 0.25) (layer "B.Cu") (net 4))
 (segment (start 116.704511 116.336767) (end 116.045789 116.995489) (width 0.25) (layer "B.Cu") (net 4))
 (segment (start 116.704511 104.004511) (end 116.704511 116.336767) (width 0.25) (layer "B.Cu") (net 4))
 (segment (start 115.58 102.88) (end 97.78 102.88) (width 0.25) (layer "B.Cu") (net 4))
 (segment (start 115.58 102.88) (end 121.94 96.52) (width 0.25) (layer "B.Cu") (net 4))
 (segment (start 111.31048 119.193803) (end 111.31048 131.63548) (width 0.25) (layer "B.Cu") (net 4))
 (segment (start 97.78 102.88) (end 96.52 104.14) (width 0.25) (layer "B.Cu") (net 4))
 (segment (start 113.508794 116.995489) (end 111.31048 119.193803) (width 0.25) (layer "B.Cu") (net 4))
 (segment (start 116.045789 116.995489) (end 113.508794 116.995489) (width 0.25) (layer "B.Cu") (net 4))
 (segment (start 123.2 138.445) (end 115.58 138.445) (width 0.25) (layer "B.Cu") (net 4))
 (segment (start 115.58 102.88) (end 116.704511 104.004511) (width 0.25) (layer "B.Cu") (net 4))
 (segment (start 149.471 96.52) (end 153.757 92.234) (width 0.25) (layer "B.Cu") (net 4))
 (segment (start 123.2 138.445) (end 123.2 135.905) (width 0.25) (layer "B.Cu") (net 4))
 (segment (start 97.79 92.71) (end 99.06 93.98) (width 0.25) (layer "F.Cu") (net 14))
 (segment (start 99.06 93.98) (end 101.6 93.98) (width 0.25) (layer "F.Cu") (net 14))
 (segment (start 101.6 93.98) (end 107.94 87.64) (width 0.25) (layer "F.Cu") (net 14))
 (segment (start 107.94 87.64) (end 115.58 87.64) (width 0.25) (layer "F.Cu") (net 14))
 (segment (start 126.254 93.234) (end 154.432 93.234) (width 0.25) (layer "F.Cu") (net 32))
 (segment (start 123.2 90.18) (end 126.254 93.234) (width 0.25) (layer "F.Cu") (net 32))
 (segment (start 97.79 100.33) (end 107.94 90.18) (width 0.25) (layer "F.Cu") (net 11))
 (segment (start 107.94 90.18) (end 115.58 90.18) (width 0.25) (layer "F.Cu") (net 11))
 (segment (start 97.79 105.41) (end 97.79 100.33) (width 0.25) (layer "F.Cu") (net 11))
 (segment (start 123.2 92.72) (end 124.714 94.234) (width 0.25) (layer "F.Cu") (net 31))
 (segment (start 124.714 94.234) (end 154.432 94.234) (width 0.25) (layer "F.Cu") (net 31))
 (segment (start 87.122 79.502) (end 85.511 79.502) (width 0.25) (layer "F.Cu") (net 35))
 (segment (start 99.06 91.44) (end 87.122 79.502) (width 0.25) (layer "F.Cu") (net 35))
 (segment (start 99.06 104.14) (end 99.06 105.447457) (width 0.25) (layer "B.Cu") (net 12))
 (segment (start 99.06 105.447457) (end 94.271457 110.236) (width 0.25) (layer "B.Cu") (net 12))
 (segment (start 94.271457 110.236) (end 86.36 110.236) (width 0.25) (layer "B.Cu") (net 12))
 (segment (start 113.305489 135.639511) (end 86.868 135.639511) (width 0.25) (layer "F.Cu") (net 3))
 (segment (start 115.58 133.365) (end 113.305489 135.639511) (width 0.25) (layer "F.Cu") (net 3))
 (segment (start 115.58 130.825) (end 111.76 127.005) (width 0.25) (layer "B.Cu") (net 2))
 (segment (start 113.02 118.12) (end 115.58 118.12) (width 0.25) (layer "B.Cu") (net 2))
 (segment (start 111.76 127.005) (end 111.76 119.38) (width 0.25) (layer "B.Cu") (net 2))
 (segment (start 111.76 119.38) (end 113.02 118.12) (width 0.25) (layer "B.Cu") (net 2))
 (segment (start 116.84 140.6747) (end 116.84 142.265) (width 0.25) (layer "F.Cu") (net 6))
 (segment (start 116.84 142.265) (end 115.58 143.525) (width 0.25) (layer "F.Cu") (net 6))
 (segment (start 124.324511 133.830789) (end 123.374811 134.780489) (width 0.25) (layer "F.Cu") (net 6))
 (segment (start 123.374811 134.780489) (end 122.734211 134.780489) (width 0.25) (layer "F.Cu") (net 6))
 (segment (start 124.324511 119.244511) (end 124.324511 133.830789) (width 0.25) (layer "F.Cu") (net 6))
 (segment (start 123.2 118.12) (end 124.324511 119.244511) (width 0.25) (layer "F.Cu") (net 6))
 (segment (start 122.734211 134.780489) (end 116.84 140.6747) (width 0.25) (layer "F.Cu") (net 6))
 (segment (start 124.324511 142.400489) (end 123.2 143.525) (width 0.25) (layer "B.Cu") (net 7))
 (segment (start 123.2 115.58) (end 124.324511 116.704511) (width 0.25) (layer "B.Cu") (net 7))
 (segment (start 124.324511 116.704511) (end 124.324511 142.400489) (width 0.25) (layer "B.Cu") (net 7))
 (segment (start 123.2 130.825) (end 122.075489 129.700489) (width 0.25) (layer "F.Cu") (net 10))
 (segment (start 122.075489 129.695489) (end 119.38 127) (width 0.25) (layer "F.Cu") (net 10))
 (segment (start 119.38 116.86) (end 123.2 113.04) (width 0.25) (layer "F.Cu") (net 10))
 (segment (start 122.075489 129.700489) (end 122.075489 129.695489) (width 0.25) (layer "F.Cu") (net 10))
 (segment (start 119.38 127) (end 119.38 116.86) (width 0.25) (layer "F.Cu") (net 10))
 (segment (start 85.011978 78.502) (end 84.761489 78.752489) (width 0.25) (layer "F.Cu") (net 1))
 (segment (start 85.511 78.502) (end 85.011978 78.502) (width 0.25) (layer "F.Cu") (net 1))
 (segment (start 96.781489 109.486489) (end 86.614 109.486489) (width 0.25) (layer "F.Cu") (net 1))
 (segment (start 115.58 128.285) (end 96.781489 109.486489) (width 0.25) (layer "F.Cu") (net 1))
 (segment (start 84.761489 78.752489) (end 84.761489 107.637489) (width 0.25) (layer "F.Cu") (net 1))
 (segment (start 84.761489 107.637489) (end 86.36 109.236) (width 0.25) (layer "F.Cu") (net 1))
 (segment (start 149.812 151.55) (end 128.685 151.55) (width 0.25) (layer "F.Cu") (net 1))
 (segment (start 128.685 151.55) (end 123.2 146.065) (width 0.25) (layer "F.Cu") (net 1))
 (segment (start 115.58 146.065) (end 123.2 146.065) (width 0.25) (layer "B.Cu") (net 1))
 (segment (start 115.58 128.285) (end 123.2 128.285) (width 0.25) (layer "B.Cu") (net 1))
 (segment (start 124.766 96.234) (end 154.432 96.234) (width 0.25) (layer "F.Cu") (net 29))
 (segment (start 123.2 97.8) (end 124.766 96.234) (width 0.25) (layer "F.Cu") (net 29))
 (segment (start 123.2 95.26) (end 154.406 95.26) (width 0.25) (layer "F.Cu") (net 30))
 (segment (start 154.406 95.26) (end 154.432 95.234) (width 0.25) (layer "F.Cu") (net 30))
 (segment (start 121.784511 139.569511) (end 114.931511 139.569511) (width 0.25) (layer "B.Cu") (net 8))
 (segment (start 123.2 140.985) (end 121.784511 139.569511) (width 0.25) (layer "B.Cu") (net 8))
 (segment (start 110.252 134.89) (end 86.973 134.89) (width 0.25) (layer "B.Cu") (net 8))
 (segment (start 114.931511 139.569511) (end 110.252 134.89) (width 0.25) (layer "B.Cu") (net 8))
 (segment (start 122.075489 132.240489) (end 88.622511 132.240489) (width 0.25) (layer "F.Cu") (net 9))
 (segment (start 88.622511 132.240489) (end 86.973 133.89) (width 0.25) (layer "F.Cu") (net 9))
 (segment (start 123.2 133.365) (end 122.075489 132.240489) (width 0.25) (layer "F.Cu") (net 9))
 (segment (start 111.485 136.89) (end 86.973 136.89) (width 0.25) (layer "B.Cu") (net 5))
 (segment (start 115.58 140.985) (end 111.485 136.89) (width 0.25) (layer "B.Cu") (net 5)))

